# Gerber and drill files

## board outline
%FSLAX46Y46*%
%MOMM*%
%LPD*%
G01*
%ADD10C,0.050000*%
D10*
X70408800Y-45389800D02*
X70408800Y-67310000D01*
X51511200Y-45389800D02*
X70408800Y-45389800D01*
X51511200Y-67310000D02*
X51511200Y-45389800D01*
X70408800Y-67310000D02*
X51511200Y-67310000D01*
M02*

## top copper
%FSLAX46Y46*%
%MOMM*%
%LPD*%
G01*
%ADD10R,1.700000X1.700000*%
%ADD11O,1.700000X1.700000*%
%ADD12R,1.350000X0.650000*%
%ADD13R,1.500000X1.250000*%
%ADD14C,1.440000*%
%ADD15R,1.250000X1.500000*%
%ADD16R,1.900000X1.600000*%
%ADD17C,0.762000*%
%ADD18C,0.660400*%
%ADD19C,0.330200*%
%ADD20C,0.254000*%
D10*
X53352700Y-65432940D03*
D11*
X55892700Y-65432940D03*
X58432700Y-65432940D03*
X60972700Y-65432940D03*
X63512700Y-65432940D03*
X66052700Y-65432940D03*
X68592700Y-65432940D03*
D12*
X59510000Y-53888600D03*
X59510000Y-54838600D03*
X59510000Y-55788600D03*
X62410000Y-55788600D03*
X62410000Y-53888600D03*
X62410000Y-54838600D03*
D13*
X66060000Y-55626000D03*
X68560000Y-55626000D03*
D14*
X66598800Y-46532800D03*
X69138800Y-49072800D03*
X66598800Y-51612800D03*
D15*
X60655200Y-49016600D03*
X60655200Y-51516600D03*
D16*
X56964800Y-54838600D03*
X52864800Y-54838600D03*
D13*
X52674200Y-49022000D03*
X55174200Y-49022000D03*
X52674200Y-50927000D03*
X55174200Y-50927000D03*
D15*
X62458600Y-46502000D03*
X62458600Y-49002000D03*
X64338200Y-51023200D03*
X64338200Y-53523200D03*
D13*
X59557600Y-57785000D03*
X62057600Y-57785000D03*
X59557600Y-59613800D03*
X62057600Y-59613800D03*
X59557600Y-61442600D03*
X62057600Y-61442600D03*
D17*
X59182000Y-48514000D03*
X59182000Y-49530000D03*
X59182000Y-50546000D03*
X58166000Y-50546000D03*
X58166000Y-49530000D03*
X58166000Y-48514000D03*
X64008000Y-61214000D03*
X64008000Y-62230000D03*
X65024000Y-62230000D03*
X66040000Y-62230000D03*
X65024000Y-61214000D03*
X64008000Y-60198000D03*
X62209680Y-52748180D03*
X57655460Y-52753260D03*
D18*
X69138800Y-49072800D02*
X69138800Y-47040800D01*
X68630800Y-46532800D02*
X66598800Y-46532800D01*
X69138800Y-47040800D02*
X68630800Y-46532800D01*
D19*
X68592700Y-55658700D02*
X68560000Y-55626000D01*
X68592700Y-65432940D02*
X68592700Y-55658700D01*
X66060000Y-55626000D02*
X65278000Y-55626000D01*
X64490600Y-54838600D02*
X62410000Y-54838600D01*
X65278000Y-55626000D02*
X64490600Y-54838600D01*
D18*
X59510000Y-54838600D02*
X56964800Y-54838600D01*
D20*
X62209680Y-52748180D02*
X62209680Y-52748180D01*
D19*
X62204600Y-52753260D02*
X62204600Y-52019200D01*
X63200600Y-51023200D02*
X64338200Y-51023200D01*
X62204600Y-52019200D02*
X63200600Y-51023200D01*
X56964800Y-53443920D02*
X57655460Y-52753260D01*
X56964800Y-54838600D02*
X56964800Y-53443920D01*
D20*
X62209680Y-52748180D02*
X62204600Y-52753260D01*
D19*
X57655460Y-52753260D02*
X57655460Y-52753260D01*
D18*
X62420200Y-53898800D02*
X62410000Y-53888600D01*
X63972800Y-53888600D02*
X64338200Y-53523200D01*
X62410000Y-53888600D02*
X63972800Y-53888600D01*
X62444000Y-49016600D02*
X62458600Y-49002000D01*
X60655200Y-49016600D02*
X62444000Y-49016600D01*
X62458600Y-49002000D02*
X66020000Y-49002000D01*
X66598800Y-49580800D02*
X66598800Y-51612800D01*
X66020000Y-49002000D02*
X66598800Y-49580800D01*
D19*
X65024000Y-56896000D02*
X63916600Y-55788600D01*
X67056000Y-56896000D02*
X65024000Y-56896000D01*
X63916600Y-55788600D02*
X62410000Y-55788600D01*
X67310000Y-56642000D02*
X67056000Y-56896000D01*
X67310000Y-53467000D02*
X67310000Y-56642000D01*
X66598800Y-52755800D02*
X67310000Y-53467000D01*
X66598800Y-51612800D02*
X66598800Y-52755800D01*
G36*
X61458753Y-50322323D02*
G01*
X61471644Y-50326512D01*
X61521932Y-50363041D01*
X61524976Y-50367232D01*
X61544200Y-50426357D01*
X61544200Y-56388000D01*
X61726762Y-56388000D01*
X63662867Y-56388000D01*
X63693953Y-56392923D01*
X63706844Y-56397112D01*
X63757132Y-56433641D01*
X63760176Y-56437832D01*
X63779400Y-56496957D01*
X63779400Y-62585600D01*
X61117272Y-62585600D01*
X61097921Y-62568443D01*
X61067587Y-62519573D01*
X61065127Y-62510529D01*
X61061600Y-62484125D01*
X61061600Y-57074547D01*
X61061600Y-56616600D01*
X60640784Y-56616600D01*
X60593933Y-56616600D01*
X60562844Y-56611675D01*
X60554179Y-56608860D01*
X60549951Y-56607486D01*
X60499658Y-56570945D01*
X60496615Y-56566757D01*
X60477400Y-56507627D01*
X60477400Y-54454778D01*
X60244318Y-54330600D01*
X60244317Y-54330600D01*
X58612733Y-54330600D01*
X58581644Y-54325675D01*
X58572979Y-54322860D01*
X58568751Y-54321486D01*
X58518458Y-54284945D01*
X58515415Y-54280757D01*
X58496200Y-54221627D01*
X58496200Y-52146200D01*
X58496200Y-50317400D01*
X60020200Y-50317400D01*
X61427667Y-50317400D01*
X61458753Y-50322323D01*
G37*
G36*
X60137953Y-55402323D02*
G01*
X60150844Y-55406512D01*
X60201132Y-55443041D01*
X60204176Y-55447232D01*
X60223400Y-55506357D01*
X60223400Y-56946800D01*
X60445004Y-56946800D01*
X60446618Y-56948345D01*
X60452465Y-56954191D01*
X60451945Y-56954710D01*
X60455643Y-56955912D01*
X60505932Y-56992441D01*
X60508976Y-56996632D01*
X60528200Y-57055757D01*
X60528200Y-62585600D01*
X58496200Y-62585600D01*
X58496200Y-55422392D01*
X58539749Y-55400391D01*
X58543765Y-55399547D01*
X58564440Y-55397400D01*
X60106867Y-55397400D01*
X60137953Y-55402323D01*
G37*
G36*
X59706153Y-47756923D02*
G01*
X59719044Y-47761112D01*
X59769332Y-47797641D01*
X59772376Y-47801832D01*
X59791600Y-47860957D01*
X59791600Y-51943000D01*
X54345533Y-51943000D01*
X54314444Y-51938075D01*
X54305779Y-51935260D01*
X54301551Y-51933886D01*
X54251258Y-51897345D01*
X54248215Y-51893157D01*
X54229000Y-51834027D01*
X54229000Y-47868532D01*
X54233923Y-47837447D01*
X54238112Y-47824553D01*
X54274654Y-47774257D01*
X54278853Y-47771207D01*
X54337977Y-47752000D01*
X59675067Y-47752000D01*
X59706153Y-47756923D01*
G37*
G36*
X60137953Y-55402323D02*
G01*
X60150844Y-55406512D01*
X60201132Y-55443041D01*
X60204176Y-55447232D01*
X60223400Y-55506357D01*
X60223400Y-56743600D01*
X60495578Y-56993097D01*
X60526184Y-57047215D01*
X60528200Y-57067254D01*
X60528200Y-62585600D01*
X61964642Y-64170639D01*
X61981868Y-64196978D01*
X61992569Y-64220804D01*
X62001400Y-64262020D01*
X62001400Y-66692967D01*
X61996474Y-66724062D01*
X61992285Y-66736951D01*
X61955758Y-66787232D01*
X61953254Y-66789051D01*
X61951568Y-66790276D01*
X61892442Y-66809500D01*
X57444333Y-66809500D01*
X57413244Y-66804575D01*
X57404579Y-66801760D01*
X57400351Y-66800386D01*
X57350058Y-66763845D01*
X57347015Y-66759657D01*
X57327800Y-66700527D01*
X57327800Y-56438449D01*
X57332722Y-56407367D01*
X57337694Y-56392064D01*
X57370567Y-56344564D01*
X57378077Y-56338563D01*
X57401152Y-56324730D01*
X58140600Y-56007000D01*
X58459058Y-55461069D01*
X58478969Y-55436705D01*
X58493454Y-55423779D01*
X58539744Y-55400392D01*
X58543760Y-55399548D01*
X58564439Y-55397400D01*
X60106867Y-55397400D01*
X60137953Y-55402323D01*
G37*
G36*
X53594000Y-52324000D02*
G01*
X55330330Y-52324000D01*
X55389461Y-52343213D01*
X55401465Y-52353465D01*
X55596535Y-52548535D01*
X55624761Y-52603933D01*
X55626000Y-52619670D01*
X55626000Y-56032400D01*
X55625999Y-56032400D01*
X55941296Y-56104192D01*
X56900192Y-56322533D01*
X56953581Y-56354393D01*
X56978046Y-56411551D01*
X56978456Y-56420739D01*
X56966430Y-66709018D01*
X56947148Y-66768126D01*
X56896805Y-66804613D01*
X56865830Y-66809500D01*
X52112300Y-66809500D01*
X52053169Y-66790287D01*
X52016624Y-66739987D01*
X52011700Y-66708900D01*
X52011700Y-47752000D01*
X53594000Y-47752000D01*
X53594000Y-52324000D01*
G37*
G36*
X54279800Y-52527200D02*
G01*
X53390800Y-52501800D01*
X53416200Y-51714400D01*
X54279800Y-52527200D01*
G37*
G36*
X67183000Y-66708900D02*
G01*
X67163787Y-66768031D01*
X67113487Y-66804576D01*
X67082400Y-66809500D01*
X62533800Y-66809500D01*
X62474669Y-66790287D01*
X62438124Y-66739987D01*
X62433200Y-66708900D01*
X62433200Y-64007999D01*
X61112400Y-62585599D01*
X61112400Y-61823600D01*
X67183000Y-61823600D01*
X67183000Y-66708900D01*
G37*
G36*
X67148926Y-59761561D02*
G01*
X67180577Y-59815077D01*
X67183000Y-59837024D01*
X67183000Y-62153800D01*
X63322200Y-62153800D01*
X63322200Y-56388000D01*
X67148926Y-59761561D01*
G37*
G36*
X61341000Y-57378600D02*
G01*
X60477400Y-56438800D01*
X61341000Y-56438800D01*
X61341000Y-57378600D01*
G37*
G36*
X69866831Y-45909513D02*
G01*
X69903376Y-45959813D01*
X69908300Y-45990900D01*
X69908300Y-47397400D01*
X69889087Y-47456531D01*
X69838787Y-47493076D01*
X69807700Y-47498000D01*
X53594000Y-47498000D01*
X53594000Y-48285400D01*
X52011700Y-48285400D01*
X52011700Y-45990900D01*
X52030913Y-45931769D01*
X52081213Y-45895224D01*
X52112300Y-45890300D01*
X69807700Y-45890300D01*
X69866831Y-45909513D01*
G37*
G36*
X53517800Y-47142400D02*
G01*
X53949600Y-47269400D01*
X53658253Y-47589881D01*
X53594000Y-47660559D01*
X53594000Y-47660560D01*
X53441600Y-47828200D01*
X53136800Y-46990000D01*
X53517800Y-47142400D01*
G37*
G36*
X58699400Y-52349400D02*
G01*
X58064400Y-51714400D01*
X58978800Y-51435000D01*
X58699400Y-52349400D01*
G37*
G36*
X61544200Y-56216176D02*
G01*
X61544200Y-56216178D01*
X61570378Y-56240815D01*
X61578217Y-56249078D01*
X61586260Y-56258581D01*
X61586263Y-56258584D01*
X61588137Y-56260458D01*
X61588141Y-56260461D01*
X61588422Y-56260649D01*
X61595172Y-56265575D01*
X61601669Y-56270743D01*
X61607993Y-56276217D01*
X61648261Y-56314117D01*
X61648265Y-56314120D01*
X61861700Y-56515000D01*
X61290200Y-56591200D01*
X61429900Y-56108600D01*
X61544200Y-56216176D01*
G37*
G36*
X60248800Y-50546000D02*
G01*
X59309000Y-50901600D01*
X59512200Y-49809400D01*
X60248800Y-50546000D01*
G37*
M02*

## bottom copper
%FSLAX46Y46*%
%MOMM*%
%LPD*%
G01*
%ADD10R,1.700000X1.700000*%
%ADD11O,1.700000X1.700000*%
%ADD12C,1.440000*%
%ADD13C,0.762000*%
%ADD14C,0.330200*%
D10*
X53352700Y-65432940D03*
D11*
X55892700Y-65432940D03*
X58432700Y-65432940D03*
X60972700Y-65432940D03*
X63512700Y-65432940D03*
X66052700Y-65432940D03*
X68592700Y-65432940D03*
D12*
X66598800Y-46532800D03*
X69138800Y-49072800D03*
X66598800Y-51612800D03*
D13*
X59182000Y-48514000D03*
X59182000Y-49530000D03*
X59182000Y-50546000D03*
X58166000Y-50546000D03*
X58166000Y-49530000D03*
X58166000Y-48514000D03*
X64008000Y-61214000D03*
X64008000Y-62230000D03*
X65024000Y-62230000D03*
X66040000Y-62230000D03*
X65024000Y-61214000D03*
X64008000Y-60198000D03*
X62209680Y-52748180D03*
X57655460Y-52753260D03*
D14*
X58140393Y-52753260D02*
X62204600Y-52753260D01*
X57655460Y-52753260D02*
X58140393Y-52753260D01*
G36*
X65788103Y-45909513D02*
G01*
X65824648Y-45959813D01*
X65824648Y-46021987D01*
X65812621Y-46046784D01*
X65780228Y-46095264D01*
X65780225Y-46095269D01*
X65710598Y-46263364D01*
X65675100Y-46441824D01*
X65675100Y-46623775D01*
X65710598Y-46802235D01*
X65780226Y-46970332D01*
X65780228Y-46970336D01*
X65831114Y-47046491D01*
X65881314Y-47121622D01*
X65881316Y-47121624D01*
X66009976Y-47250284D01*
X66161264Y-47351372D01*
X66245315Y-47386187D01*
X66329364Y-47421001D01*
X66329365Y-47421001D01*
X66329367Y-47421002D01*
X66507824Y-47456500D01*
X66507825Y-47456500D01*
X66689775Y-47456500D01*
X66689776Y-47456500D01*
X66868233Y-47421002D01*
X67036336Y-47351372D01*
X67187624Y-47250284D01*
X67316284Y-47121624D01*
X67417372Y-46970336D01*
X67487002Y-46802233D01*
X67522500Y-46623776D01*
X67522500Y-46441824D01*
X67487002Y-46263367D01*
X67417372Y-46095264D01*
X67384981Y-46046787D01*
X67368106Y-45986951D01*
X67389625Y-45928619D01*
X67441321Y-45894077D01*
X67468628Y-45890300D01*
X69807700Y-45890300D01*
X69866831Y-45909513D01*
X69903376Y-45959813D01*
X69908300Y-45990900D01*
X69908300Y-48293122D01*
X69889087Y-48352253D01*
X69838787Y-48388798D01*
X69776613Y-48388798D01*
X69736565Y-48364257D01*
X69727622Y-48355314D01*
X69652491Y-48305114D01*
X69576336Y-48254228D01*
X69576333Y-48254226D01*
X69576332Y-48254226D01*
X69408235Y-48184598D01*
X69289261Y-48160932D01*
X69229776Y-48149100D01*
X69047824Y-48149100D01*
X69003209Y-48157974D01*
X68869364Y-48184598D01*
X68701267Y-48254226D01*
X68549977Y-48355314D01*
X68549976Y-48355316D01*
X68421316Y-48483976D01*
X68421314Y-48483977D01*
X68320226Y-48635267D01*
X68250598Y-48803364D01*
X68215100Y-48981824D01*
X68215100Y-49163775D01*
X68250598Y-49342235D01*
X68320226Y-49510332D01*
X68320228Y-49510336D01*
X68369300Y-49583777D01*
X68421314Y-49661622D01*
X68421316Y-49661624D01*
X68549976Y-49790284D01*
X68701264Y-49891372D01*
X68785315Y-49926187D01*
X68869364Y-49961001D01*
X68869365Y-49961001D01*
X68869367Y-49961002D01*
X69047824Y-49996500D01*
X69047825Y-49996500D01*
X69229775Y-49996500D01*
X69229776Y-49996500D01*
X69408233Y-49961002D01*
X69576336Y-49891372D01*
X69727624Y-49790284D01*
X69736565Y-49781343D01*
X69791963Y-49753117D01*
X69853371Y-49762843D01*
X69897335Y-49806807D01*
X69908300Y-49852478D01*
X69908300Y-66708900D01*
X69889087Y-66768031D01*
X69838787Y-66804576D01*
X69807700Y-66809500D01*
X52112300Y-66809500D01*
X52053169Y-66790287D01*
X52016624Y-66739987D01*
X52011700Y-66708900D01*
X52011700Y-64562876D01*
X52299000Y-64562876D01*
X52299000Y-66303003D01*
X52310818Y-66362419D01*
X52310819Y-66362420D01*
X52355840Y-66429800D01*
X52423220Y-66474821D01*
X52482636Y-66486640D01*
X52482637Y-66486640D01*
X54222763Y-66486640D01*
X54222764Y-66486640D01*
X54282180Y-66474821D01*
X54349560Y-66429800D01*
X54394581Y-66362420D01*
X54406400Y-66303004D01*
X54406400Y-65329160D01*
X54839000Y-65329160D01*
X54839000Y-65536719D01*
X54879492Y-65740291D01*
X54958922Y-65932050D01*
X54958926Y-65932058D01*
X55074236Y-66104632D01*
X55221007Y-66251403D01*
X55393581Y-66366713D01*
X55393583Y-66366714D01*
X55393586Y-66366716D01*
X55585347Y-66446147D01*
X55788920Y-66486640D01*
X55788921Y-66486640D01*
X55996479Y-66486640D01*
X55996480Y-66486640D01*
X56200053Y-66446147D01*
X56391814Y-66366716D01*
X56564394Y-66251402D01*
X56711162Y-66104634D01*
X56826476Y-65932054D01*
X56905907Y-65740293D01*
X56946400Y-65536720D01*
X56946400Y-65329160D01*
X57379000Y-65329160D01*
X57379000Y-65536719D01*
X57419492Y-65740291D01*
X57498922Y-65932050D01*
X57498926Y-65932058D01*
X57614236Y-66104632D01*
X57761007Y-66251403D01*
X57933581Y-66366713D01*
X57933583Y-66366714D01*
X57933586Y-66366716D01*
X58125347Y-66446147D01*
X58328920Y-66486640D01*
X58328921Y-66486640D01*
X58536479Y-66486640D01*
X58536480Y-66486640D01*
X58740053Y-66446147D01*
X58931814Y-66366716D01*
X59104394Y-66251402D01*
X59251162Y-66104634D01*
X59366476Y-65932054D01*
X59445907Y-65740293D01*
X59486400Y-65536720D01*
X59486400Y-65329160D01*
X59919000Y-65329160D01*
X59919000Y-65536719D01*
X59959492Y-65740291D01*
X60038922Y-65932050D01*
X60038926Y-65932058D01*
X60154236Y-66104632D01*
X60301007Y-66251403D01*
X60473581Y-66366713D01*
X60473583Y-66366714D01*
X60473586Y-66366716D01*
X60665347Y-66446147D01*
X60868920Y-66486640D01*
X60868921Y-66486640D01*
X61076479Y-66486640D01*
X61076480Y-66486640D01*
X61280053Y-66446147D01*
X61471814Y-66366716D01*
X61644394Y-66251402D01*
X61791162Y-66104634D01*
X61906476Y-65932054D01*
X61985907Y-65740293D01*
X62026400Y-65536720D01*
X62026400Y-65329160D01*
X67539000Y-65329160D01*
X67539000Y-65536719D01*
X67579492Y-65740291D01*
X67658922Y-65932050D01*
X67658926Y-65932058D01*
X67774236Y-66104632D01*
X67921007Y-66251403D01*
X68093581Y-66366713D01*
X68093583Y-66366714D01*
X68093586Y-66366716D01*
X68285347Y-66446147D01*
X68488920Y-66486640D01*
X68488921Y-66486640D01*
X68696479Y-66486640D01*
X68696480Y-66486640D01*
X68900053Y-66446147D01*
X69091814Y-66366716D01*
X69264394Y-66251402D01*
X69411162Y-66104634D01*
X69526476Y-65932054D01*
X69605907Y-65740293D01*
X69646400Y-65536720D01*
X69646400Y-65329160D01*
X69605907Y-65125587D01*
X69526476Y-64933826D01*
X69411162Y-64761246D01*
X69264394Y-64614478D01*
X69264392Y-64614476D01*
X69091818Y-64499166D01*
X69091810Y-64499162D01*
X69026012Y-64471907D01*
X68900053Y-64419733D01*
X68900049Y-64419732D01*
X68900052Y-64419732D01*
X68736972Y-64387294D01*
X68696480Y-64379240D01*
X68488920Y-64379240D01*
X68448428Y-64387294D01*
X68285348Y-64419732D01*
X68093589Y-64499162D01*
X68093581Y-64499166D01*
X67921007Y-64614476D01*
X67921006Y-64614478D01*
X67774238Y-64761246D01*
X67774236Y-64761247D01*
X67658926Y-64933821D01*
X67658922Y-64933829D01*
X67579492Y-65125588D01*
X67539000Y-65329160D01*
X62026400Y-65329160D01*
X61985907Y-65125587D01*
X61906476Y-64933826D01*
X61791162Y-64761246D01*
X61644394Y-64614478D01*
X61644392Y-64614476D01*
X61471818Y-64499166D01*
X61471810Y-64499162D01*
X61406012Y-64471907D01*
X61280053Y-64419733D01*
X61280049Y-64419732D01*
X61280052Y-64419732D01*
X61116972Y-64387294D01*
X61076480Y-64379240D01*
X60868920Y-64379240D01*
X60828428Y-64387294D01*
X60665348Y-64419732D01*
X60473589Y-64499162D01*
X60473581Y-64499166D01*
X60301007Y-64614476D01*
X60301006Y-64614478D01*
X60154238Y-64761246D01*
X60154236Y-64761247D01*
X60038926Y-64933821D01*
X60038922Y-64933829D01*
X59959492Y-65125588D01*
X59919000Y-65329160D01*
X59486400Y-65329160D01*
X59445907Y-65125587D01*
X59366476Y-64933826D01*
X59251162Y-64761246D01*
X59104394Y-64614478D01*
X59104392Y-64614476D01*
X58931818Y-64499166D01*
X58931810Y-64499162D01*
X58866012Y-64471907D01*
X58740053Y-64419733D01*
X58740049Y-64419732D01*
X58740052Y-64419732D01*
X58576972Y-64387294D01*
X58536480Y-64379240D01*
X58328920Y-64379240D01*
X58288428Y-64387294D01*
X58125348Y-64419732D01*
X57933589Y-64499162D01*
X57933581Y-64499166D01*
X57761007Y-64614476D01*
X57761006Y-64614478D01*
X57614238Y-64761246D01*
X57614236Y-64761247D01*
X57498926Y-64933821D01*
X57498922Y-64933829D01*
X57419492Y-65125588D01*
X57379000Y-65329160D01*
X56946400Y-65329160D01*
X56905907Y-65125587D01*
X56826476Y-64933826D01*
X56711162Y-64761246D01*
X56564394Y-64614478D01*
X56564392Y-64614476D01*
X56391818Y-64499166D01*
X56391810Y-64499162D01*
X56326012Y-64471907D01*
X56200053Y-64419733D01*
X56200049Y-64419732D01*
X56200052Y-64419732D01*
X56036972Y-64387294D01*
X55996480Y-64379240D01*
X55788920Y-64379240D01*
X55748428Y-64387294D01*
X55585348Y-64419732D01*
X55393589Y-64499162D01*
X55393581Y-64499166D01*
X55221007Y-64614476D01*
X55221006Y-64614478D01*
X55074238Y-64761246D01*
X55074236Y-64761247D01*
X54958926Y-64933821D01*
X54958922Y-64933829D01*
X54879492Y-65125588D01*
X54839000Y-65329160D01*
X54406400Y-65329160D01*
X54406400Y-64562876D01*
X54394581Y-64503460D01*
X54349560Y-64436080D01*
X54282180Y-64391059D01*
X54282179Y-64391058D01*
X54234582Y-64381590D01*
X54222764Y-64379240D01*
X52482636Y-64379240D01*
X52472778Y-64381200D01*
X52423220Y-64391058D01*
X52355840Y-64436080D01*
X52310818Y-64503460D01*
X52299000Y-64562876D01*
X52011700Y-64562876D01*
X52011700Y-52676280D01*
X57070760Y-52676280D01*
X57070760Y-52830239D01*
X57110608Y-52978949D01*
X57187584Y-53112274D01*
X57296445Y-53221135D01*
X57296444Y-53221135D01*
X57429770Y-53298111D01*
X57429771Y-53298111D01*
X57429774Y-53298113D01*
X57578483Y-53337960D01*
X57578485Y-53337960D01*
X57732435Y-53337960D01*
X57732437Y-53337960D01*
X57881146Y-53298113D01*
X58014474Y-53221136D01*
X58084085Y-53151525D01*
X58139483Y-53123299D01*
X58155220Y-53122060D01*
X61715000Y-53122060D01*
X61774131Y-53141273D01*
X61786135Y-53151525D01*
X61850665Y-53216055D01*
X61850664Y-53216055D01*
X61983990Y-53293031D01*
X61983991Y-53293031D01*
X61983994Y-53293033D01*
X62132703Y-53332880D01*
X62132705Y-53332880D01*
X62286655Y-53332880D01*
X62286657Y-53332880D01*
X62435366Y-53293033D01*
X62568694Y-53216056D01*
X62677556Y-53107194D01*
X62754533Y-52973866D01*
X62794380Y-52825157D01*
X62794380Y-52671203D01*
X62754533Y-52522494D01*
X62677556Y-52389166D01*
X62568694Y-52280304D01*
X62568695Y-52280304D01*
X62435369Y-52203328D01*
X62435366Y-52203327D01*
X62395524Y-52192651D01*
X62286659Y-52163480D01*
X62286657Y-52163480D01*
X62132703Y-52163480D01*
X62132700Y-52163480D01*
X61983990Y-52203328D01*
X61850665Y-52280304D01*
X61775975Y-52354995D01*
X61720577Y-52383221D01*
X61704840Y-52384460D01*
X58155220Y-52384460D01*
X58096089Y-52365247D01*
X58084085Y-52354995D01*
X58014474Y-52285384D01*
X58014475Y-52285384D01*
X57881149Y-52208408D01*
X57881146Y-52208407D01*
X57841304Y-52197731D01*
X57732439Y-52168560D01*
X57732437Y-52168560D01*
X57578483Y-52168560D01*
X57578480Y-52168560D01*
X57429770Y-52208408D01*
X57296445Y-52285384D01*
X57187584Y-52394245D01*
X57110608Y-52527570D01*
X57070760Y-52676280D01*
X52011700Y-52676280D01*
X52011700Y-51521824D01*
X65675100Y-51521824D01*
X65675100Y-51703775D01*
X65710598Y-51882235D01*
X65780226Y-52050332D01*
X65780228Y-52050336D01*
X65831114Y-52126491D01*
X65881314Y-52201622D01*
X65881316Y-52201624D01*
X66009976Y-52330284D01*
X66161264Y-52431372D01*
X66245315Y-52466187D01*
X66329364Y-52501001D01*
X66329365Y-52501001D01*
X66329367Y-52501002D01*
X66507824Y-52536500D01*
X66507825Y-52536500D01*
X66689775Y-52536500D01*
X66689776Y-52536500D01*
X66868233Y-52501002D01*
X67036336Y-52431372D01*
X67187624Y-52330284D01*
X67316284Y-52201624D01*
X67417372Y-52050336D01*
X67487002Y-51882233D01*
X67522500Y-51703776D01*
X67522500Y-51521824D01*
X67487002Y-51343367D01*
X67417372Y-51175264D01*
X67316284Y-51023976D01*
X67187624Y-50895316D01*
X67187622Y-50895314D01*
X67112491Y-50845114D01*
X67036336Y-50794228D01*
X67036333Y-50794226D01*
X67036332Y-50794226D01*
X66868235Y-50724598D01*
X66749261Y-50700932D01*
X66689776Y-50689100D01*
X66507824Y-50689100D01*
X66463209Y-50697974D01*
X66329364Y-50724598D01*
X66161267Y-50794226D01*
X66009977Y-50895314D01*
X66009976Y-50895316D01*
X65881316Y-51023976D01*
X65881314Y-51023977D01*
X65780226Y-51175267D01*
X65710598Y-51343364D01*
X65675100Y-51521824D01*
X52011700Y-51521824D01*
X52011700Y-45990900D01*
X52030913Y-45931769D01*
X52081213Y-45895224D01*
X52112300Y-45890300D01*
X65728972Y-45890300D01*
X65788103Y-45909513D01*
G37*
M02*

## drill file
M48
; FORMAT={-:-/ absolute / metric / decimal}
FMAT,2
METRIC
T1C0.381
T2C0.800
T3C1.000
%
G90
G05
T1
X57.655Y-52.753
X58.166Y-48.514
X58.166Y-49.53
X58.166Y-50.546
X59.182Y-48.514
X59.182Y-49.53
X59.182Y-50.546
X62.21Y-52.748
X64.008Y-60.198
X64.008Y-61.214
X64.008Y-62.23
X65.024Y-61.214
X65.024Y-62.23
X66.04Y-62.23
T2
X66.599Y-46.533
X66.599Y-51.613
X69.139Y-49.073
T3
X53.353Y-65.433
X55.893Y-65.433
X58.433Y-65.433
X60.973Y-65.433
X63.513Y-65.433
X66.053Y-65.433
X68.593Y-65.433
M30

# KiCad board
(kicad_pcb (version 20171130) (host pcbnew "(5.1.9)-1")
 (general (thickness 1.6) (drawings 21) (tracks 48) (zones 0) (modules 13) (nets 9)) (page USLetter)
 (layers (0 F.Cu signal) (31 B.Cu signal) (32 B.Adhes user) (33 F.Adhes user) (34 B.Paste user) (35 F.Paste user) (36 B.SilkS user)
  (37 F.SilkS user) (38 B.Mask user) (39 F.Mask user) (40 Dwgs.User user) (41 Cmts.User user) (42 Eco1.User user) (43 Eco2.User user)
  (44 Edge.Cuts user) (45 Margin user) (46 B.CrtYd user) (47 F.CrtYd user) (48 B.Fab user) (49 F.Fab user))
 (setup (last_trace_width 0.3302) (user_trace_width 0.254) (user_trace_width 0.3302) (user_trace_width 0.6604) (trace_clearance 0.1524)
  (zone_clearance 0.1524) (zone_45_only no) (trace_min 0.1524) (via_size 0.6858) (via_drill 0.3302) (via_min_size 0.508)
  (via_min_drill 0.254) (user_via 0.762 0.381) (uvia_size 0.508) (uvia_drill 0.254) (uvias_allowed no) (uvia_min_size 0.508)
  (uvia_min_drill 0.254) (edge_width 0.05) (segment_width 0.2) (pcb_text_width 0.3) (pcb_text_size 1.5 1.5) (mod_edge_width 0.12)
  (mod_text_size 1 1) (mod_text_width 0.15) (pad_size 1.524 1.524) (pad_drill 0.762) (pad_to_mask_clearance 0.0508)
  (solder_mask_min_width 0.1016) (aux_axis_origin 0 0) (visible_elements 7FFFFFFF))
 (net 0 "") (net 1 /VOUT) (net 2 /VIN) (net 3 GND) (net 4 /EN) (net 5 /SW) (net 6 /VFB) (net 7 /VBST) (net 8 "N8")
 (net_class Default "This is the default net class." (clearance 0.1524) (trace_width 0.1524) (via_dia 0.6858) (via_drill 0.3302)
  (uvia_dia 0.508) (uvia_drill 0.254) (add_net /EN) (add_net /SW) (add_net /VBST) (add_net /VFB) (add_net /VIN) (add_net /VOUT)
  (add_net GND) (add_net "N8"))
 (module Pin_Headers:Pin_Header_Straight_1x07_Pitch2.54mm (layer F.Cu) (at 53.3527 65.43294 90)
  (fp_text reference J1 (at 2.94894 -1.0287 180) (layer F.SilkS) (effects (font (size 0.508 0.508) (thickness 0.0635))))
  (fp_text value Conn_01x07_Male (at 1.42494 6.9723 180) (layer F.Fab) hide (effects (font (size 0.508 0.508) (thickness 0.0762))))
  (pad 1 thru_hole rect (at 0 0 90) (size 1.7 1.7) (drill 1) (layers *.Cu *.Mask) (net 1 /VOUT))
  (pad 2 thru_hole oval (at 0 2.54 90) (size 1.7 1.7) (drill 1) (layers *.Cu *.Mask) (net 1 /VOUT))
  (pad 3 thru_hole oval (at 0 5.08 90) (size 1.7 1.7) (drill 1) (layers *.Cu *.Mask) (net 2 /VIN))
  (pad 4 thru_hole oval (at 0 7.62 90) (size 1.7 1.7) (drill 1) (layers *.Cu *.Mask) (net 2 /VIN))
  (pad 5 thru_hole oval (at 0 10.16 90) (size 1.7 1.7) (drill 1) (layers *.Cu *.Mask) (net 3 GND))
  (pad 6 thru_hole oval (at 0 12.7 90) (size 1.7 1.7) (drill 1) (layers *.Cu *.Mask) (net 3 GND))
  (pad 7 thru_hole oval (at 0 15.24 90) (size 1.7 1.7) (drill 1) (layers *.Cu *.Mask) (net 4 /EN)))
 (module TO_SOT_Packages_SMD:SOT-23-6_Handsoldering (layer F.Cu) (at 60.96 54.8386)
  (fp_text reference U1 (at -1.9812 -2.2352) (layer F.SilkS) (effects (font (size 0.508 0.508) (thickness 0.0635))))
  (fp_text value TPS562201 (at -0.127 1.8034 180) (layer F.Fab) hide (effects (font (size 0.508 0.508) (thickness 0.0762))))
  (pad 1 smd rect (at -1.45 -0.95) (size 1.35 0.65) (layers F.Cu F.Paste F.Mask) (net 3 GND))
  (pad 2 smd rect (at -1.45 0) (size 1.35 0.65) (layers F.Cu F.Paste F.Mask) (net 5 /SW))
  (pad 3 smd rect (at -1.45 0.95) (size 1.35 0.65) (layers F.Cu F.Paste F.Mask) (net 2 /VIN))
  (pad 4 smd rect (at 1.45 0.95) (size 1.35 0.65) (layers F.Cu F.Paste F.Mask) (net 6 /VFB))
  (pad 6 smd rect (at 1.45 -0.95) (size 1.35 0.65) (layers F.Cu F.Paste F.Mask) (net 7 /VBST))
  (pad 5 smd rect (at 1.45 0) (size 1.35 0.65) (layers F.Cu F.Paste F.Mask) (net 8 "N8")))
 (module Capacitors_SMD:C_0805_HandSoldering (layer F.Cu) (at 67.31 55.626)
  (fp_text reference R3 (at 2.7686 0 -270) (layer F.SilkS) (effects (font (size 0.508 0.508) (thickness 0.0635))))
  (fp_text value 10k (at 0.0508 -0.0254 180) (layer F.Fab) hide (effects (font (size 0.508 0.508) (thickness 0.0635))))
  (pad 1 smd rect (at -1.25 0) (size 1.5 1.25) (layers F.Cu F.Paste F.Mask) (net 8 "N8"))
  (pad 2 smd rect (at 1.25 0) (size 1.5 1.25) (layers F.Cu F.Paste F.Mask) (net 4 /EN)))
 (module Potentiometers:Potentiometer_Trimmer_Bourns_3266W (layer F.Cu) (at 66.5988 46.5328 90)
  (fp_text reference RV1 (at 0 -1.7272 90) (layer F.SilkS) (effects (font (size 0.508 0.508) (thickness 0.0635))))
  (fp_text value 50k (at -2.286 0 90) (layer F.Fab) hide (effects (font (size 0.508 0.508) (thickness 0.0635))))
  (pad 1 thru_hole circle (at 0 0 90) (size 1.44 1.44) (drill 0.8) (layers *.Cu *.Mask) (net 1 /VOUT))
  (pad 2 thru_hole circle (at -2.54 2.54 90) (size 1.44 1.44) (drill 0.8) (layers *.Cu *.Mask) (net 1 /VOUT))
  (pad 3 thru_hole circle (at -5.08 0 90) (size 1.44 1.44) (drill 0.8) (layers *.Cu *.Mask) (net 6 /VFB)))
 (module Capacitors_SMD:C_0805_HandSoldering (layer F.Cu) (at 60.6552 50.2666 270)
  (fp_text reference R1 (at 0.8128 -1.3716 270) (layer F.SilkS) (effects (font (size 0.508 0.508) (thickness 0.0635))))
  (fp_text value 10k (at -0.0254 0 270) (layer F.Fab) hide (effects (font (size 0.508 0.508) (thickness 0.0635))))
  (pad 1 smd rect (at -1.25 0 270) (size 1.5 1.25) (layers F.Cu F.Paste F.Mask) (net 6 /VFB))
  (pad 2 smd rect (at 1.25 0 270) (size 1.5 1.25) (layers F.Cu F.Paste F.Mask) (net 3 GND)))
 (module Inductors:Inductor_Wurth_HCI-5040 (layer F.Cu) (at 54.9148 54.8386 180)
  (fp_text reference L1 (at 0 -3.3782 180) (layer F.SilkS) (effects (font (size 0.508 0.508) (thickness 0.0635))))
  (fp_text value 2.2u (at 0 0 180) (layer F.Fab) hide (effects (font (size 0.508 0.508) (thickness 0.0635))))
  (pad 1 smd rect (at -2.05 0 180) (size 1.9 1.6) (layers F.Cu F.Paste F.Mask) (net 5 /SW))
  (pad 2 smd rect (at 2.05 0 180) (size 1.9 1.6) (layers F.Cu F.Paste F.Mask) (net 1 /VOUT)))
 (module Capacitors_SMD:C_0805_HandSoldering (layer F.Cu) (at 53.9242 49.022)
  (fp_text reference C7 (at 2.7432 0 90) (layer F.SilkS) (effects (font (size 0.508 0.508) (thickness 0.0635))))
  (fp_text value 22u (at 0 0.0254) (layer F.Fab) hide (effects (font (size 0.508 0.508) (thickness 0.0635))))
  (pad 1 smd rect (at -1.25 0) (size 1.5 1.25) (layers F.Cu F.Paste F.Mask) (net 1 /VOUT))
  (pad 2 smd rect (at 1.25 0) (size 1.5 1.25) (layers F.Cu F.Paste F.Mask) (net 3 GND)))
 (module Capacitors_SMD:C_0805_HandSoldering (layer F.Cu) (at 53.9242 50.927)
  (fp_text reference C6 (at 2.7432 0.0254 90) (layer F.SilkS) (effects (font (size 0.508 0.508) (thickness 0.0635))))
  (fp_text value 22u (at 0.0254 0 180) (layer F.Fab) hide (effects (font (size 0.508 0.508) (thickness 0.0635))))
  (pad 1 smd rect (at -1.25 0) (size 1.5 1.25) (layers F.Cu F.Paste F.Mask) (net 1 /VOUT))
  (pad 2 smd rect (at 1.25 0) (size 1.5 1.25) (layers F.Cu F.Paste F.Mask) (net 3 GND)))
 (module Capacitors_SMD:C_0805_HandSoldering (layer F.Cu) (at 62.4586 47.752 270)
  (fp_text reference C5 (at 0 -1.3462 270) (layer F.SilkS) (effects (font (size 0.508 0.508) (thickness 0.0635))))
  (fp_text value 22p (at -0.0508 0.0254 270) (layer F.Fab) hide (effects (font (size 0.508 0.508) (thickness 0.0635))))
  (pad 1 smd rect (at -1.25 0 270) (size 1.5 1.25) (layers F.Cu F.Paste F.Mask) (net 1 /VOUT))
  (pad 2 smd rect (at 1.25 0 270) (size 1.5 1.25) (layers F.Cu F.Paste F.Mask) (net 6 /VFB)))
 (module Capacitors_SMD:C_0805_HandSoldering (layer F.Cu) (at 64.3382 52.2732 270)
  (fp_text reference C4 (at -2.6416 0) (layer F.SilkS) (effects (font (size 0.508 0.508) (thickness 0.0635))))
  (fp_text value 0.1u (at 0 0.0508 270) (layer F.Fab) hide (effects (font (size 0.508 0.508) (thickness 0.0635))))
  (pad 1 smd rect (at -1.25 0 270) (size 1.5 1.25) (layers F.Cu F.Paste F.Mask) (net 5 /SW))
  (pad 2 smd rect (at 1.25 0 270) (size 1.5 1.25) (layers F.Cu F.Paste F.Mask) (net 7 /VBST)))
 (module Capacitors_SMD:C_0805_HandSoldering (layer F.Cu) (at 60.8076 57.785)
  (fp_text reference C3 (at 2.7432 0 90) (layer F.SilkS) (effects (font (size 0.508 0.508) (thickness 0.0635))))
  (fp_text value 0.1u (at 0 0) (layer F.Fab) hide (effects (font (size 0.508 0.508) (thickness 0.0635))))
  (pad 1 smd rect (at -1.25 0) (size 1.5 1.25) (layers F.Cu F.Paste F.Mask) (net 2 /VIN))
  (pad 2 smd rect (at 1.25 0) (size 1.5 1.25) (layers F.Cu F.Paste F.Mask) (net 3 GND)))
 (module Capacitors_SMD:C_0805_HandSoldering (layer F.Cu) (at 60.8076 59.6138)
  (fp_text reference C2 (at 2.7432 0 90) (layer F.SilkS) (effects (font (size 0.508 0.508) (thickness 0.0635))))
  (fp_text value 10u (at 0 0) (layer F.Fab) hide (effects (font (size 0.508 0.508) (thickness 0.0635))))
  (pad 1 smd rect (at -1.25 0) (size 1.5 1.25) (layers F.Cu F.Paste F.Mask) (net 2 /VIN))
  (pad 2 smd rect (at 1.25 0) (size 1.5 1.25) (layers F.Cu F.Paste F.Mask) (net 3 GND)))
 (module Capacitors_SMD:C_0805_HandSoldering (layer F.Cu) (at 60.8076 61.4426)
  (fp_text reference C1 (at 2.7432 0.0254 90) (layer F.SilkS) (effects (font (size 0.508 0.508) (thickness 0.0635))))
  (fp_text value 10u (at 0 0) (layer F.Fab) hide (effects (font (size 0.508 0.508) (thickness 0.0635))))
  (pad 1 smd rect (at -1.25 0) (size 1.5 1.25) (layers F.Cu F.Paste F.Mask) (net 2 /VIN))
  (pad 2 smd rect (at 1.25 0) (size 1.5 1.25) (layers F.Cu F.Paste F.Mask) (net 3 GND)))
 (gr_line (start 70.4088 45.3898) (end 70.4088 67.31) (layer Edge.Cuts) (width 0.05))
 (gr_line (start 51.5112 45.3898) (end 70.4088 45.3898) (layer Edge.Cuts) (width 0.05))
 (gr_line (start 51.5112 67.31) (end 51.5112 45.3898) (layer Edge.Cuts) (width 0.05))
 (gr_line (start 70.4088 67.31) (end 51.5112 67.31) (layer Edge.Cuts) (width 0.05))
 (via (at 59.182 48.514) (size 0.762) (drill 0.381) (layers F.Cu B.Cu) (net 3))
 (via (at 59.182 49.53) (size 0.762) (drill 0.381) (layers F.Cu B.Cu) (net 3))
 (via (at 59.182 50.546) (size 0.762) (drill 0.381) (layers F.Cu B.Cu) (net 3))
 (via (at 58.166 50.546) (size 0.762) (drill 0.381) (layers F.Cu B.Cu) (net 3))
 (via (at 58.166 49.53) (size 0.762) (drill 0.381) (layers F.Cu B.Cu) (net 3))
 (via (at 58.166 48.514) (size 0.762) (drill 0.381) (layers F.Cu B.Cu) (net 3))
 (via (at 64.008 61.214) (size 0.762) (drill 0.381) (layers F.Cu B.Cu) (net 3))
 (via (at 64.008 62.23) (size 0.762) (drill 0.381) (layers F.Cu B.Cu) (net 3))
 (via (at 65.024 62.23) (size 0.762) (drill 0.381) (layers F.Cu B.Cu) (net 3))
 (via (at 66.04 62.23) (size 0.762) (drill 0.381) (layers F.Cu B.Cu) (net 3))
 (via (at 65.024 61.214) (size 0.762) (drill 0.381) (layers F.Cu B.Cu) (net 3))
 (via (at 64.008 60.198) (size 0.762) (drill 0.381) (layers F.Cu B.Cu) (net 3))
 (segment (start 69.1388 49.0728) (end 69.1388 47.0408) (width 0.6604) (layer F.Cu) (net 1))
 (segment (start 68.6308 46.5328) (end 66.5988 46.5328) (width 0.6604) (layer F.Cu) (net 1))
 (segment (start 69.1388 47.0408) (end 68.6308 46.5328) (width 0.6604) (layer F.Cu) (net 1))
 (segment (start 68.5927 55.6587) (end 68.56 55.626) (width 0.3302) (layer F.Cu) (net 4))
 (segment (start 68.5927 65.43294) (end 68.5927 55.6587) (width 0.3302) (layer F.Cu) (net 4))
 (segment (start 66.06 55.626) (end 65.278 55.626) (width 0.3302) (layer F.Cu) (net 8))
 (segment (start 64.4906 54.8386) (end 62.41 54.8386) (width 0.3302) (layer F.Cu) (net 8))
 (segment (start 65.278 55.626) (end 64.4906 54.8386) (width 0.3302) (layer F.Cu) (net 8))
 (segment (start 59.51 54.8386) (end 56.9648 54.8386) (width 0.6604) (layer F.Cu) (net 5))
 (segment (start 62.20968 52.74818) (end 62.20968 52.74818) (width 0.254) (layer F.Cu) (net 5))
 (segment (start 62.2046 52.75326) (end 62.2046 52.0192) (width 0.3302) (layer F.Cu) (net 5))
 (segment (start 63.2006 51.0232) (end 64.3382 51.0232) (width 0.3302) (layer F.Cu) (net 5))
 (segment (start 62.2046 52.0192) (end 63.2006 51.0232) (width 0.3302) (layer F.Cu) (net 5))
 (segment (start 56.9648 53.44392) (end 57.65546 52.75326) (width 0.3302) (layer F.Cu) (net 5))
 (segment (start 56.9648 54.8386) (end 56.9648 53.44392) (width 0.3302) (layer F.Cu) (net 5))
 (segment (start 58.140393 52.75326) (end 62.2046 52.75326) (width 0.3302) (layer B.Cu) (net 5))
 (segment (start 57.65546 52.75326) (end 58.140393 52.75326) (width 0.3302) (layer B.Cu) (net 5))
 (segment (start 62.20968 52.74818) (end 62.2046 52.75326) (width 0.254) (layer F.Cu) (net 5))
 (via (at 62.20968 52.74818) (size 0.762) (drill 0.381) (layers F.Cu B.Cu) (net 5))
 (segment (start 57.65546 52.75326) (end 57.65546 52.75326) (width 0.3302) (layer F.Cu) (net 5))
 (via (at 57.65546 52.75326) (size 0.762) (drill 0.381) (layers F.Cu B.Cu) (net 5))
 (segment (start 62.4202 53.8988) (end 62.41 53.8886) (width 0.6604) (layer F.Cu) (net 7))
 (segment (start 63.9728 53.8886) (end 64.3382 53.5232) (width 0.6604) (layer F.Cu) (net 7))
 (segment (start 62.41 53.8886) (end 63.9728 53.8886) (width 0.6604) (layer F.Cu) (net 7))
 (segment (start 62.444 49.0166) (end 62.4586 49.002) (width 0.6604) (layer F.Cu) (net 6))
 (segment (start 60.6552 49.0166) (end 62.444 49.0166) (width 0.6604) (layer F.Cu) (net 6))
 (segment (start 62.4586 49.002) (end 66.02 49.002) (width 0.6604) (layer F.Cu) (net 6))
 (segment (start 66.5988 49.5808) (end 66.5988 51.6128) (width 0.6604) (layer F.Cu) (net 6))
 (segment (start 66.02 49.002) (end 66.5988 49.5808) (width 0.6604) (layer F.Cu) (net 6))
 (segment (start 65.024 56.896) (end 63.9166 55.7886) (width 0.3302) (layer F.Cu) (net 6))
 (segment (start 67.056 56.896) (end 65.024 56.896) (width 0.3302) (layer F.Cu) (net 6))
 (segment (start 63.9166 55.7886) (end 62.41 55.7886) (width 0.3302) (layer F.Cu) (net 6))
 (segment (start 67.31 56.642) (end 67.056 56.896) (width 0.3302) (layer F.Cu) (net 6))
 (segment (start 67.31 53.467) (end 67.31 56.642) (width 0.3302) (layer F.Cu) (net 6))
 (segment (start 66.5988 52.7558) (end 67.31 53.467) (width 0.3302) (layer F.Cu) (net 6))
 (segment (start 66.5988 51.6128) (end 66.5988 52.7558) (width 0.3302) (layer F.Cu) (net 6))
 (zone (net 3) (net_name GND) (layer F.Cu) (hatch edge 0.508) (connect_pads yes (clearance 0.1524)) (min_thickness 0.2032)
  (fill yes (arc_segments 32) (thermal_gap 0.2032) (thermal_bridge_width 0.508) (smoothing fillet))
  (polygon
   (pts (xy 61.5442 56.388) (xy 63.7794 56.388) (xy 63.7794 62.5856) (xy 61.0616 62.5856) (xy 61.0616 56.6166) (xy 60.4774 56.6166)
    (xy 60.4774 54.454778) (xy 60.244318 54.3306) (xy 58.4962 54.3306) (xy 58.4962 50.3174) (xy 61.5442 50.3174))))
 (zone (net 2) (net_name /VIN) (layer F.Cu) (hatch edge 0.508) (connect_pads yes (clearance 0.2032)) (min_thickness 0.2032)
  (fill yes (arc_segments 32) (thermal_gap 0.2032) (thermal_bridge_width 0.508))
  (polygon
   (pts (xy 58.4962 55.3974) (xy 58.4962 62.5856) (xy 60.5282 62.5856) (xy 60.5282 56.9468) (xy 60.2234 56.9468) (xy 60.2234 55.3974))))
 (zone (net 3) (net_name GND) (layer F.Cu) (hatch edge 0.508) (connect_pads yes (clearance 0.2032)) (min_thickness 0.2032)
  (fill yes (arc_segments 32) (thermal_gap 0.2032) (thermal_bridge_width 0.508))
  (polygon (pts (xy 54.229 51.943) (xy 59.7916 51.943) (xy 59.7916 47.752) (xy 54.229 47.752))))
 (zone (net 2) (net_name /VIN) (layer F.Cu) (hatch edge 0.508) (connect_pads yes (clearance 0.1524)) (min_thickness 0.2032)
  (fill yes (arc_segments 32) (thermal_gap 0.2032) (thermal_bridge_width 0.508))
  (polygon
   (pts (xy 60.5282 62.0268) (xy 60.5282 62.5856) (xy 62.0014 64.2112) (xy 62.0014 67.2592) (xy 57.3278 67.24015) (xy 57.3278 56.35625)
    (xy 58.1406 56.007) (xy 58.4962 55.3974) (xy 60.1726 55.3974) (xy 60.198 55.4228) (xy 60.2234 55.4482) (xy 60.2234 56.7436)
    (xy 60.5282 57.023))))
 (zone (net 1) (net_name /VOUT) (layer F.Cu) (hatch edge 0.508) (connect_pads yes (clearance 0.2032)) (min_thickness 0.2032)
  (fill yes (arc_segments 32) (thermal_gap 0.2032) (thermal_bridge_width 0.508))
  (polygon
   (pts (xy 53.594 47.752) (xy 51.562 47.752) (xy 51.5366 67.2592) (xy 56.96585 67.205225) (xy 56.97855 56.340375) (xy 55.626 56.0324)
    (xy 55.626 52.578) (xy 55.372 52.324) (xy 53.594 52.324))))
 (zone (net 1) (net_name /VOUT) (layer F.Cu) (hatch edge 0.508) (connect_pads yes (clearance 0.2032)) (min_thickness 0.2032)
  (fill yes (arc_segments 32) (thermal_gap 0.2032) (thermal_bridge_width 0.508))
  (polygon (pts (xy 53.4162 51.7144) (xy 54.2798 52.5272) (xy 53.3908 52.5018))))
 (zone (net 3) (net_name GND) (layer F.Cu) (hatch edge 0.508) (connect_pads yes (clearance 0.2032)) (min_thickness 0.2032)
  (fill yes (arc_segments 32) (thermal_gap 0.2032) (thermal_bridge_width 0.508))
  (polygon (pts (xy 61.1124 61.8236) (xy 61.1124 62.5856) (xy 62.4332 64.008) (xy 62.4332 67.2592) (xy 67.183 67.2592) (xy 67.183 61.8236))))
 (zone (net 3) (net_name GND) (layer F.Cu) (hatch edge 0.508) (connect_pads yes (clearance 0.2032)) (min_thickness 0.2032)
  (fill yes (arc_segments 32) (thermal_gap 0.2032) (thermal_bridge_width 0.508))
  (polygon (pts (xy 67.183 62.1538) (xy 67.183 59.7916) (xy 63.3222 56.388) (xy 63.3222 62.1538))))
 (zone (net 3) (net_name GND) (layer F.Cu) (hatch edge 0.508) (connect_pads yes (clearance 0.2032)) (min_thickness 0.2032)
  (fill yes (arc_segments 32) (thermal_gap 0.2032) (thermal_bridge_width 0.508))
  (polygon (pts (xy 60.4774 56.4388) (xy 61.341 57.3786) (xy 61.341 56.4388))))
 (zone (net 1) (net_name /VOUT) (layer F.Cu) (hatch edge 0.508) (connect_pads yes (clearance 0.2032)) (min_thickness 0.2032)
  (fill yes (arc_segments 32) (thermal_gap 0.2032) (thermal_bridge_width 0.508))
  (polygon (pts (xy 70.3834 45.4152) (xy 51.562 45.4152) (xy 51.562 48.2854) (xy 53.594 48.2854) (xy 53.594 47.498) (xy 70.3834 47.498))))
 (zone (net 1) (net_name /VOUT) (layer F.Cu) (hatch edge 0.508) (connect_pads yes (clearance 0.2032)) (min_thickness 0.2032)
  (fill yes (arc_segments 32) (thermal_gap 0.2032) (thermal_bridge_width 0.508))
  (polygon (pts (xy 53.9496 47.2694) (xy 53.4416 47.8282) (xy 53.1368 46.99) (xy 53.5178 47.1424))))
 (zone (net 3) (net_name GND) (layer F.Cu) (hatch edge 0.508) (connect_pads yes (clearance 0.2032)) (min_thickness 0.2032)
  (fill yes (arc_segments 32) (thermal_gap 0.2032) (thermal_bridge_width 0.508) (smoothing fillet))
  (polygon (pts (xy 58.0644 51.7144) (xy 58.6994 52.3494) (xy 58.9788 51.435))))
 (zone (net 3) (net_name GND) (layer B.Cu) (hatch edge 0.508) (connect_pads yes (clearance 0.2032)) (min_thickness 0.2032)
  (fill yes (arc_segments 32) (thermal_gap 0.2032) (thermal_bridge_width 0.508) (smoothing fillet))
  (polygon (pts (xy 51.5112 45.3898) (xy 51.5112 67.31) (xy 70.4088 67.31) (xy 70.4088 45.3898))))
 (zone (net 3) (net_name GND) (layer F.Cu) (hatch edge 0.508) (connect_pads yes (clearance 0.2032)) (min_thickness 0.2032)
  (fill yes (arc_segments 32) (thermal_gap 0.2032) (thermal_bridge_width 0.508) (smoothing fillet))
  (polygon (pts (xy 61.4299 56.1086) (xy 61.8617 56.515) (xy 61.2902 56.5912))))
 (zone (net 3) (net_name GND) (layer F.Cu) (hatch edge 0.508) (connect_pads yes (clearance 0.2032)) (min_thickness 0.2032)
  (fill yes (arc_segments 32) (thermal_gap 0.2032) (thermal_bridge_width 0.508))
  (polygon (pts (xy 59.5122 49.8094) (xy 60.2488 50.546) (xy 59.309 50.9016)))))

